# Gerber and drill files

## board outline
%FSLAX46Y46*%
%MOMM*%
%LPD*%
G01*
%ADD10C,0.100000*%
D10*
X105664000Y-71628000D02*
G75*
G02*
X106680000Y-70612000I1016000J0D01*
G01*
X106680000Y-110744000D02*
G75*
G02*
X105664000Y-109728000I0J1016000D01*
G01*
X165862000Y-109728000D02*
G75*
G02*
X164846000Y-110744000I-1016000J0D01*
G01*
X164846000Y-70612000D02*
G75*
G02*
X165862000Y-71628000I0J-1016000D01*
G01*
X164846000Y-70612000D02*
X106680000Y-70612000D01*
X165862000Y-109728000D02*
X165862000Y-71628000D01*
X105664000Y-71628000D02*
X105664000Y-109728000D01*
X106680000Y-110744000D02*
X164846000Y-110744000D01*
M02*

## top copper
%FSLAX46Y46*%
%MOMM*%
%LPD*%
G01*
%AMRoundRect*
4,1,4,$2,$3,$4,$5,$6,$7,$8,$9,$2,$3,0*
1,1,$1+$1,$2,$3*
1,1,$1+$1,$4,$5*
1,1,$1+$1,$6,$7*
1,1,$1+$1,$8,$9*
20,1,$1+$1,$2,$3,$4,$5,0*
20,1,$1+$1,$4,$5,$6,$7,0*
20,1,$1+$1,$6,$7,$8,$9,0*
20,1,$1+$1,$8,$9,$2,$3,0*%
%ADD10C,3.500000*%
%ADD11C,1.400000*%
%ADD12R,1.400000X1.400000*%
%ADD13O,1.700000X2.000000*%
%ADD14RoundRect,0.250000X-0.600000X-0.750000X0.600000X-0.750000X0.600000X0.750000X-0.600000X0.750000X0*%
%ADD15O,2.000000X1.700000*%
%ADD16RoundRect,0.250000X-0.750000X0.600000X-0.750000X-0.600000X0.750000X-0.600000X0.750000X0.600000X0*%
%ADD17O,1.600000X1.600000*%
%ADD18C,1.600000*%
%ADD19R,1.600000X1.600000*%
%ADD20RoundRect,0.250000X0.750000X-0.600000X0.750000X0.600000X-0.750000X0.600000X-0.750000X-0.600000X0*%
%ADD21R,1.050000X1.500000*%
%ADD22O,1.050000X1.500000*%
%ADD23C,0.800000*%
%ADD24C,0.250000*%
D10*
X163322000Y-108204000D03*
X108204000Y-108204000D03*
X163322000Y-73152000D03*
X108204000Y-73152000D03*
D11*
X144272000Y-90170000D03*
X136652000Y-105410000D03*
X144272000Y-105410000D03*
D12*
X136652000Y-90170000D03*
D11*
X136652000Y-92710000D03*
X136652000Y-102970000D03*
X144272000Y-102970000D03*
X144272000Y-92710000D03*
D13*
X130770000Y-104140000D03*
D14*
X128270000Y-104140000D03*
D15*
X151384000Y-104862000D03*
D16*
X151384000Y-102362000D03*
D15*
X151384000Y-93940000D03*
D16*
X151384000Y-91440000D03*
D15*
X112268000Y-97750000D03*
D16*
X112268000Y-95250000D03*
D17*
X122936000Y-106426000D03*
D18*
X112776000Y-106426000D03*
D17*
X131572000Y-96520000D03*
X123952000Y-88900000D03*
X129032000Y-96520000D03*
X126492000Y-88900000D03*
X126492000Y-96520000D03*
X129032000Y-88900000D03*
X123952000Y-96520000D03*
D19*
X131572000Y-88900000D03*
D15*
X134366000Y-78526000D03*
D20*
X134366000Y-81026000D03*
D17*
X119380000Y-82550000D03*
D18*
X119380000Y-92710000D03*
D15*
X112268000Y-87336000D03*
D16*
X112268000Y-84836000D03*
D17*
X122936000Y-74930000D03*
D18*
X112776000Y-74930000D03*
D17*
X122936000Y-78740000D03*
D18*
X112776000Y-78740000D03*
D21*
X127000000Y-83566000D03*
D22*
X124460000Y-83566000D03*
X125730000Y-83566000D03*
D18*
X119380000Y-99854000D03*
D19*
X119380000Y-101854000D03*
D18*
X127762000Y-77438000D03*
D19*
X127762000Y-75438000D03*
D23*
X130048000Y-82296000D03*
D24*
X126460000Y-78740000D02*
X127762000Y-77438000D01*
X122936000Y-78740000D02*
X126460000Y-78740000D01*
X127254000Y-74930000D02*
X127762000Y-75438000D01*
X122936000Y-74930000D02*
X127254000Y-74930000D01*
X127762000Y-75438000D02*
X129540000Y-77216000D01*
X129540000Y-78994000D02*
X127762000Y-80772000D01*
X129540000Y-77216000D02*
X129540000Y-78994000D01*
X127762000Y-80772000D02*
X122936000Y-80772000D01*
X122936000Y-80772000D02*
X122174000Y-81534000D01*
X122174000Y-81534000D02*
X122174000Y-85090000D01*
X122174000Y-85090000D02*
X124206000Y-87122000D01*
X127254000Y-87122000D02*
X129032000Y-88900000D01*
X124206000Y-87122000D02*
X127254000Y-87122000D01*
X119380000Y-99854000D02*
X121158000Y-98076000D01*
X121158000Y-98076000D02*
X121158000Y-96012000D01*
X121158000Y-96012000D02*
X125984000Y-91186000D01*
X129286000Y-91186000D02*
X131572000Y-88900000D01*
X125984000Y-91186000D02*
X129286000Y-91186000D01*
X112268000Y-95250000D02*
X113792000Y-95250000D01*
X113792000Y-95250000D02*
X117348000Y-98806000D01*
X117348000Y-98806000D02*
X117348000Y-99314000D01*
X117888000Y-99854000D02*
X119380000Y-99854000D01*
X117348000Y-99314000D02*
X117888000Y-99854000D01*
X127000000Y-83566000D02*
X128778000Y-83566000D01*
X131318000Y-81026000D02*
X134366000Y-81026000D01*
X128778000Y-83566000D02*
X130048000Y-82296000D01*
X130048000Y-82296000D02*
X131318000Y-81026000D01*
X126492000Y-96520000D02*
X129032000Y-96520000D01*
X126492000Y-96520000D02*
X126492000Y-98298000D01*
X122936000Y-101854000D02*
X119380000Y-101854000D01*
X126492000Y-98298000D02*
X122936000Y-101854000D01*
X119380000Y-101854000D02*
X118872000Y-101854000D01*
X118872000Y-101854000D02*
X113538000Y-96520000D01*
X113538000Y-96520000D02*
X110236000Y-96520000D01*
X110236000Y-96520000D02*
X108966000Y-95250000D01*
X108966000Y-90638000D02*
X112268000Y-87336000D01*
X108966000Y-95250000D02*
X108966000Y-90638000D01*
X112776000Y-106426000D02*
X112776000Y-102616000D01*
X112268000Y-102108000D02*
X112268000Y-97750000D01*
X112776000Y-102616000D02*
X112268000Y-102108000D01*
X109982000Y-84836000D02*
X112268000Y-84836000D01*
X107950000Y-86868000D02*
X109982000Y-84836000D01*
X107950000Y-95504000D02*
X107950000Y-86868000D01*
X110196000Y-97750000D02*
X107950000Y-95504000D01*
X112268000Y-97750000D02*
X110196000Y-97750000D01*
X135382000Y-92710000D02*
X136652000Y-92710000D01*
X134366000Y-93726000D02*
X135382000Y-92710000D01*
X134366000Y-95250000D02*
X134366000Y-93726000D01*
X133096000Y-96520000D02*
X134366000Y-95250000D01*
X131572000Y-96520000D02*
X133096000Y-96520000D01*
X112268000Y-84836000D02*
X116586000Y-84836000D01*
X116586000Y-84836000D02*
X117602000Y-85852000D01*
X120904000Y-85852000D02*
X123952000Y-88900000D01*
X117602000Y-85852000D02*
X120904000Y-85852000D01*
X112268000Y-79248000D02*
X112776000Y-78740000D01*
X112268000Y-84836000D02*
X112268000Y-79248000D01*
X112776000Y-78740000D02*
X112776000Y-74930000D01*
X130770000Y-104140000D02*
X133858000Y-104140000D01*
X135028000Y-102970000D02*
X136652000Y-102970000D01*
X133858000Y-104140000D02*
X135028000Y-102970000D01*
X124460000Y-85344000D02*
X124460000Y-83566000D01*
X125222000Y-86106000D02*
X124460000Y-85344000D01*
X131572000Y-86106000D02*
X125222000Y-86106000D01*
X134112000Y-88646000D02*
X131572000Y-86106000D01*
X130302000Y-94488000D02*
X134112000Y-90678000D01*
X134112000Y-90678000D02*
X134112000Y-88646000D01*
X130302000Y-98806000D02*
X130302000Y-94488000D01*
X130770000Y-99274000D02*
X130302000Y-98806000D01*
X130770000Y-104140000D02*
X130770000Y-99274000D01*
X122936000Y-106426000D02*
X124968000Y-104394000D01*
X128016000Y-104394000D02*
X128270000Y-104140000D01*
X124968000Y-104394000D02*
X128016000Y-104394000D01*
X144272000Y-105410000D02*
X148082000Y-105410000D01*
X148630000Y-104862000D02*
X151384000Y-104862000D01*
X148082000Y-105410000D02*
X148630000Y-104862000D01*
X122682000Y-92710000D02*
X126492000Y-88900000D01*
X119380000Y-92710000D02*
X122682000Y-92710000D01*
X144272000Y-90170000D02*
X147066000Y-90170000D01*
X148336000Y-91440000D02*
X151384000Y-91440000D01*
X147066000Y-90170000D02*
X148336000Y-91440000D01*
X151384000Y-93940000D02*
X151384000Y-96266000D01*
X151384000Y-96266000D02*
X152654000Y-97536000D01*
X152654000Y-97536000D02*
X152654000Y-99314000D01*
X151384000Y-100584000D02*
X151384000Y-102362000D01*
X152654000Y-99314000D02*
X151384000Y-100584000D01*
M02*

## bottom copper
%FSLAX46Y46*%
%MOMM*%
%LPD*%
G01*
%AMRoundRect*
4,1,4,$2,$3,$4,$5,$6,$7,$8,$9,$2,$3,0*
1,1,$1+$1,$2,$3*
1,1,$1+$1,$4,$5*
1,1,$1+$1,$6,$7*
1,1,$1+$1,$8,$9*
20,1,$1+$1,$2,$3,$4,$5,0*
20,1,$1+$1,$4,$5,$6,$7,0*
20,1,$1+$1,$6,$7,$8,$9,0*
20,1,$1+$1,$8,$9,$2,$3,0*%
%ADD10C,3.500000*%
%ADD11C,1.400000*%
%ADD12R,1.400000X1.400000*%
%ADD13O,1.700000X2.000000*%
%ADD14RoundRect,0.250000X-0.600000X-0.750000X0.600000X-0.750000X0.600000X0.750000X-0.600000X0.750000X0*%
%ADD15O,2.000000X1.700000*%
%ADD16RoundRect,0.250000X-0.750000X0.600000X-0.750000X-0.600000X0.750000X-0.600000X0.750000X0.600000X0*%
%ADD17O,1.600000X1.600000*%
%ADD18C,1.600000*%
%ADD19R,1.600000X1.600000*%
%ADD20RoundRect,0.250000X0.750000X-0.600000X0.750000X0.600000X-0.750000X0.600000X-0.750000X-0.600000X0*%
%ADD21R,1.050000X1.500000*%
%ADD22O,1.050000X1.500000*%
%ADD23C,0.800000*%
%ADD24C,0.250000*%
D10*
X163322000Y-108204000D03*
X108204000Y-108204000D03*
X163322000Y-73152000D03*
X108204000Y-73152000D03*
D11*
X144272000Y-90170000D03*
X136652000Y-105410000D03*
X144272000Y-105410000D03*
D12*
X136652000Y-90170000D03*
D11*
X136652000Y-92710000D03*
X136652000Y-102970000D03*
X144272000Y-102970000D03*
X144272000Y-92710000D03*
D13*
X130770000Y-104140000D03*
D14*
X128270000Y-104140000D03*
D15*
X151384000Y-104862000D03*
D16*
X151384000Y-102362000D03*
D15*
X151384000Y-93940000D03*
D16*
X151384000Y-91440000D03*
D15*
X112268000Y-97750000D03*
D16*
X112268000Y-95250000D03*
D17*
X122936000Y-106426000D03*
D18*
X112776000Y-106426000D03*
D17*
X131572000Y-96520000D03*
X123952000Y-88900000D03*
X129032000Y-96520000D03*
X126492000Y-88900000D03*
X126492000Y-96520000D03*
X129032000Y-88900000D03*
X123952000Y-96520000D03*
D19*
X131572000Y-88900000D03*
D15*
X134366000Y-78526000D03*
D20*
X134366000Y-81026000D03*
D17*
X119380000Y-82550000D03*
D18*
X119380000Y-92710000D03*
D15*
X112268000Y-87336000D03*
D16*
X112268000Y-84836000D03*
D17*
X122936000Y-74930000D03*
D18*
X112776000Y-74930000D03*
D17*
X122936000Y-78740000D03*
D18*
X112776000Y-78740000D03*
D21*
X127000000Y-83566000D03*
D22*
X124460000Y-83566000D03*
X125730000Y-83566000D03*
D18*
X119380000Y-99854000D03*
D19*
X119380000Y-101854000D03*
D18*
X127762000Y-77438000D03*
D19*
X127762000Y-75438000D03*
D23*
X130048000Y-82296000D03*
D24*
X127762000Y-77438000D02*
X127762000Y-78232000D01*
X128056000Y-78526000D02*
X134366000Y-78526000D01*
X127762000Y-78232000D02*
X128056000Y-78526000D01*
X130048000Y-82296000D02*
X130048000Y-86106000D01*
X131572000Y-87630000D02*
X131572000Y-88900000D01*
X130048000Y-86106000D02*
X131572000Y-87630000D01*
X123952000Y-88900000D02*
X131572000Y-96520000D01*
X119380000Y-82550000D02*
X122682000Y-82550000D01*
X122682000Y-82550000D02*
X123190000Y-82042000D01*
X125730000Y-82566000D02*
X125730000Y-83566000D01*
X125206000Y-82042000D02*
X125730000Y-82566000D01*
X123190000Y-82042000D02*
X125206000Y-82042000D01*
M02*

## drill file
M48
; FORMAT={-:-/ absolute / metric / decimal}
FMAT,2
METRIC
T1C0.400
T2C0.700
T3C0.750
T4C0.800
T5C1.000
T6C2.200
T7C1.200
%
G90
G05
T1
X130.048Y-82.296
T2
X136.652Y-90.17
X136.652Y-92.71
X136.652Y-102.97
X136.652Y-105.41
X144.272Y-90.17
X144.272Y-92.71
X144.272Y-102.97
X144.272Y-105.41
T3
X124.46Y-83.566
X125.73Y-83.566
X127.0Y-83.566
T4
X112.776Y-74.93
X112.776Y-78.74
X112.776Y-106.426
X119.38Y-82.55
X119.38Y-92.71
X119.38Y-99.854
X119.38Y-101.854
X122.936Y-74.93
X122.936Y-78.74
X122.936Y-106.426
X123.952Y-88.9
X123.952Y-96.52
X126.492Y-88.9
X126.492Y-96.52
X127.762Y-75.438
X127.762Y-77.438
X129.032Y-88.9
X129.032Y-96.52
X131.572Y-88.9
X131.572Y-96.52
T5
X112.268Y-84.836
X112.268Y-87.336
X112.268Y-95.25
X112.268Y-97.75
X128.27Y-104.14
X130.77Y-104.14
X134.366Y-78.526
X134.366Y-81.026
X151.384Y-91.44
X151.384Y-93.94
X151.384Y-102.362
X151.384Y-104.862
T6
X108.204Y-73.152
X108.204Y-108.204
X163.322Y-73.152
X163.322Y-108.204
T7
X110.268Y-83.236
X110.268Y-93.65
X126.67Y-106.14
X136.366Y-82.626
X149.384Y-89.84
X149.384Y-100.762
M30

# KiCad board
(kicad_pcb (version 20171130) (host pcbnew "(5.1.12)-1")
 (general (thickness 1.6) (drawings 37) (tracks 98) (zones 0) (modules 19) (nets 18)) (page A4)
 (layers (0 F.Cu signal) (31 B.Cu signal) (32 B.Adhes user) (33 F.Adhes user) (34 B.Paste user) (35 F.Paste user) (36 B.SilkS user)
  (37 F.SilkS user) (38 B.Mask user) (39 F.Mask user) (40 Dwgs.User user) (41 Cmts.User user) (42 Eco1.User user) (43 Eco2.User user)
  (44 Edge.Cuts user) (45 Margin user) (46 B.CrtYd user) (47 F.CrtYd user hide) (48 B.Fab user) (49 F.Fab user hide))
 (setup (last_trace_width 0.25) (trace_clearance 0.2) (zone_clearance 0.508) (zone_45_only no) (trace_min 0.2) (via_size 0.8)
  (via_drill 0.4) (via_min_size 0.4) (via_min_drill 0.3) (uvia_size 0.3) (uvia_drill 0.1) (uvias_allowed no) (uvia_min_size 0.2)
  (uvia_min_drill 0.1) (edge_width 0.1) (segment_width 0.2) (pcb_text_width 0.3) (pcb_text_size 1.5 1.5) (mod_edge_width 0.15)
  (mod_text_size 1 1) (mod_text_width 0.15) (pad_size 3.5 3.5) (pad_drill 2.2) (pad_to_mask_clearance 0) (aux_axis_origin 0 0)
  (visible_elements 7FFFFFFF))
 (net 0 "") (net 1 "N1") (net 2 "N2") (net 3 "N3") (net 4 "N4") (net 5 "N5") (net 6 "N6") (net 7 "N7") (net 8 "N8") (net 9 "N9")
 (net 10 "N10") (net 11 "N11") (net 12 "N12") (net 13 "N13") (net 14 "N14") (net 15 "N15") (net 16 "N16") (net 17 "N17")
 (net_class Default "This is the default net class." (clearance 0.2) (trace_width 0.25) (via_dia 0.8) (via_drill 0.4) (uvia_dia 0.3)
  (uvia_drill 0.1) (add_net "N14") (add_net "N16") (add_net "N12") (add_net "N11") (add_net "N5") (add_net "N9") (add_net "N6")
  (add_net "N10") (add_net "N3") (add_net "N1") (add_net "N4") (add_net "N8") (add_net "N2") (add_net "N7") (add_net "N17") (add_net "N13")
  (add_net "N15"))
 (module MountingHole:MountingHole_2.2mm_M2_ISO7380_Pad (layer F.Cu) (at 163.322 108.204)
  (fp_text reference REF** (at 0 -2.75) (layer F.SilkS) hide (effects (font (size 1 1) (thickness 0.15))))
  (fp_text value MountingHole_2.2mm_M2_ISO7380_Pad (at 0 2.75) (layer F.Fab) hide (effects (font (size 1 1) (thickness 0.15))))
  (pad 1 thru_hole circle (at 0 0) (size 3.5 3.5) (drill 2.2) (layers *.Cu *.Mask)))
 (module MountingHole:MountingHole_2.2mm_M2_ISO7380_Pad (layer F.Cu) (at 108.204 108.204)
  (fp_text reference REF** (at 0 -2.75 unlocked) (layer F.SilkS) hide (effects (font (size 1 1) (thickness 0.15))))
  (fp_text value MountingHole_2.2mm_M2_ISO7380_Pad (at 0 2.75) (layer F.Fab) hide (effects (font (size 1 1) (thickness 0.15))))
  (pad 1 thru_hole circle (at 0 0) (size 3.5 3.5) (drill 2.2) (layers *.Cu *.Mask)))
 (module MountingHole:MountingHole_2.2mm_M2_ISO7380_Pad (layer F.Cu) (at 163.322 73.152)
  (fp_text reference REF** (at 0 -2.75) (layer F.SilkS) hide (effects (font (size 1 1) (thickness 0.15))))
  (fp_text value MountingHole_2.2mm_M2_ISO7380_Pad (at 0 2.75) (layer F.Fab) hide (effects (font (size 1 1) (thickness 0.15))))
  (pad 1 thru_hole circle (at 0 0) (size 3.5 3.5) (drill 2.2) (layers *.Cu *.Mask)))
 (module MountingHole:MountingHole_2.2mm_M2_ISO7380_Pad (layer F.Cu) (at 108.204 73.152)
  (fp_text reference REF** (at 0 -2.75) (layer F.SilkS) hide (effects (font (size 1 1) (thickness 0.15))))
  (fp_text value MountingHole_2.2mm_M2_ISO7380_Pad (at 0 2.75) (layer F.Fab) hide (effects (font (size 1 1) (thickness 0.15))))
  (pad 1 thru_hole circle (at 0 0) (size 3.5 3.5) (drill 2.2) (layers *.Cu *.Mask)))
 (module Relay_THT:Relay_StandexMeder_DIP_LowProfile (layer F.Cu) (at 136.652 90.17)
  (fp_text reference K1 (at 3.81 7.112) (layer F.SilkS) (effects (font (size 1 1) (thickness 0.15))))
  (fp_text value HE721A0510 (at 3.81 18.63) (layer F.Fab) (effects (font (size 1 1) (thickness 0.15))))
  (pad 14 thru_hole circle (at 7.62 0) (size 1.4 1.4) (drill 0.7) (layers *.Cu *.Mask) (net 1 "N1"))
  (pad 7 thru_hole circle (at 0 15.24) (size 1.4 1.4) (drill 0.7) (layers *.Cu *.Mask) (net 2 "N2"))
  (pad 8 thru_hole circle (at 7.62 15.24) (size 1.4 1.4) (drill 0.7) (layers *.Cu *.Mask) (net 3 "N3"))
  (pad 1 thru_hole rect (at 0 0) (size 1.4 1.4) (drill 0.7) (layers *.Cu *.Mask) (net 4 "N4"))
  (pad 2 thru_hole circle (at 0 2.54) (size 1.4 1.4) (drill 0.7) (layers *.Cu *.Mask) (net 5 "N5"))
  (pad 6 thru_hole circle (at 0 12.8) (size 1.4 1.4) (drill 0.7) (layers *.Cu *.Mask) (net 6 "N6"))
  (pad 9 thru_hole circle (at 7.62 12.8) (size 1.4 1.4) (drill 0.7) (layers *.Cu *.Mask) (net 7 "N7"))
  (pad 13 thru_hole circle (at 7.62 2.54) (size 1.4 1.4) (drill 0.7) (layers *.Cu *.Mask) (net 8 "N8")))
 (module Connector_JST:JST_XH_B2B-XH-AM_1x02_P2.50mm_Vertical (layer F.Cu) (at 128.27 104.14)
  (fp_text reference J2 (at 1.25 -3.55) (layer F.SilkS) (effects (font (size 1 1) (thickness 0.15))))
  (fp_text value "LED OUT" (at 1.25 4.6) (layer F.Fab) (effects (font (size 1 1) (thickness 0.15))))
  (pad "" np_thru_hole circle (at -1.6 2) (size 1.2 1.2) (drill 1.2) (layers *.Cu *.Mask))
  (pad 2 thru_hole oval (at 2.5 0) (size 1.7 2) (drill 1) (layers *.Cu *.Mask) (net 6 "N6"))
  (pad 1 thru_hole roundrect (at 0 0) (size 1.7 2) (drill 1) (layers *.Cu *.Mask) (roundrect_rratio 0.147059) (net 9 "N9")))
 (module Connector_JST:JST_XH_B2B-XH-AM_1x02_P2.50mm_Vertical (layer F.Cu) (at 151.384 102.362 270)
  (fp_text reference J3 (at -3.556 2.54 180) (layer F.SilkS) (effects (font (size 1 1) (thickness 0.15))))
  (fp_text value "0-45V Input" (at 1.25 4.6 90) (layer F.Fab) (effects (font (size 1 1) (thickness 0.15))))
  (pad "" np_thru_hole circle (at -1.6 2 270) (size 1.2 1.2) (drill 1.2) (layers *.Cu *.Mask))
  (pad 2 thru_hole oval (at 2.5 0 270) (size 1.7 2) (drill 1) (layers *.Cu *.Mask) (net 3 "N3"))
  (pad 1 thru_hole roundrect (at 0 0 270) (size 1.7 2) (drill 1) (layers *.Cu *.Mask) (roundrect_rratio 0.147059) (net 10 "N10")))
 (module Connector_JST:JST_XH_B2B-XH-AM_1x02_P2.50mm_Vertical (layer F.Cu) (at 151.384 91.44 270)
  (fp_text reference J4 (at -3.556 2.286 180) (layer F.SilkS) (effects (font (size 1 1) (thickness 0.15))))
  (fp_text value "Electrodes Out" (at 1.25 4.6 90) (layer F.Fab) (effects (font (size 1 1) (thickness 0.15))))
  (pad "" np_thru_hole circle (at -1.6 2 270) (size 1.2 1.2) (drill 1.2) (layers *.Cu *.Mask))
  (pad 2 thru_hole oval (at 2.5 0 270) (size 1.7 2) (drill 1) (layers *.Cu *.Mask) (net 10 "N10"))
  (pad 1 thru_hole roundrect (at 0 0 270) (size 1.7 2) (drill 1) (layers *.Cu *.Mask) (roundrect_rratio 0.147059) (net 1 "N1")))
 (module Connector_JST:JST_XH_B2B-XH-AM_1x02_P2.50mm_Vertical (layer F.Cu) (at 112.268 95.25 270)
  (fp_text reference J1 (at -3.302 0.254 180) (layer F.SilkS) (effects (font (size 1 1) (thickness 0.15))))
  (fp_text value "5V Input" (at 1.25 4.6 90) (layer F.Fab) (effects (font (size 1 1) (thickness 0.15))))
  (pad "" np_thru_hole circle (at -1.6 2 270) (size 1.2 1.2) (drill 1.2) (layers *.Cu *.Mask))
  (pad 2 thru_hole oval (at 2.5 0 270) (size 1.7 2) (drill 1) (layers *.Cu *.Mask) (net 5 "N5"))
  (pad 1 thru_hole roundrect (at 0 0 270) (size 1.7 2) (drill 1) (layers *.Cu *.Mask) (roundrect_rratio 0.147059) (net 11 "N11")))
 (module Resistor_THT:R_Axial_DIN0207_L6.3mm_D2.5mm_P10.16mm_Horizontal (layer F.Cu) (at 112.776 106.426)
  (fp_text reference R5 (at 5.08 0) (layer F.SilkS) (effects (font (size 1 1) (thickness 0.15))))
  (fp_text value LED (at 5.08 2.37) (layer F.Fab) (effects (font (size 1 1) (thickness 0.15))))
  (pad 2 thru_hole oval (at 10.16 0) (size 1.6 1.6) (drill 0.8) (layers *.Cu *.Mask) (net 9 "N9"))
  (pad 1 thru_hole circle (at 0 0) (size 1.6 1.6) (drill 0.8) (layers *.Cu *.Mask) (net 5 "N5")))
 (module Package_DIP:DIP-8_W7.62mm (layer F.Cu) (at 131.572 88.9 270)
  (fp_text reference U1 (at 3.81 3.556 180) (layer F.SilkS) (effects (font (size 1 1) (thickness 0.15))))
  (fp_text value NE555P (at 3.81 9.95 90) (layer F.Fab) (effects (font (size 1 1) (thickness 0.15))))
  (pad 8 thru_hole oval (at 7.62 0 270) (size 1.6 1.6) (drill 0.8) (layers *.Cu *.Mask) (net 5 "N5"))
  (pad 4 thru_hole oval (at 0 7.62 270) (size 1.6 1.6) (drill 0.8) (layers *.Cu *.Mask) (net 5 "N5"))
  (pad 7 thru_hole oval (at 7.62 2.54 270) (size 1.6 1.6) (drill 0.8) (layers *.Cu *.Mask) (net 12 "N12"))
  (pad 3 thru_hole oval (at 0 5.08 270) (size 1.6 1.6) (drill 0.8) (layers *.Cu *.Mask) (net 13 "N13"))
  (pad 6 thru_hole oval (at 7.62 5.08 270) (size 1.6 1.6) (drill 0.8) (layers *.Cu *.Mask) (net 12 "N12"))
  (pad 2 thru_hole oval (at 0 2.54 270) (size 1.6 1.6) (drill 0.8) (layers *.Cu *.Mask) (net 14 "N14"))
  (pad 5 thru_hole oval (at 7.62 7.62 270) (size 1.6 1.6) (drill 0.8) (layers *.Cu *.Mask) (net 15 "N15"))
  (pad 1 thru_hole rect (at 0 0 270) (size 1.6 1.6) (drill 0.8) (layers *.Cu *.Mask) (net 11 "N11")))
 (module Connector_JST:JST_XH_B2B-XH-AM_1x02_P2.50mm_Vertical (layer F.Cu) (at 134.366 81.026 90)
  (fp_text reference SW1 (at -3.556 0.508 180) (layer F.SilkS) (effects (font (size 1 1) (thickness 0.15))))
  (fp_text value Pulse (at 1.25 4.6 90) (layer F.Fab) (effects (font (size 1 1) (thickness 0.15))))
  (pad "" np_thru_hole circle (at -1.6 2 90) (size 1.2 1.2) (drill 1.2) (layers *.Cu *.Mask))
  (pad 2 thru_hole oval (at 2.5 0 90) (size 1.7 2) (drill 1) (layers *.Cu *.Mask) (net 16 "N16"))
  (pad 1 thru_hole roundrect (at 0 0 90) (size 1.7 2) (drill 1) (layers *.Cu *.Mask) (roundrect_rratio 0.147059) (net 11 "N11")))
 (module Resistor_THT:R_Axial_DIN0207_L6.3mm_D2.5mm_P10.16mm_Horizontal (layer F.Cu) (at 119.38 92.71 90)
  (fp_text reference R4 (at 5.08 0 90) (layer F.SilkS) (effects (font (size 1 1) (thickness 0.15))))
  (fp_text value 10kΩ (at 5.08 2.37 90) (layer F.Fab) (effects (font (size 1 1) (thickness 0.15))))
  (pad 2 thru_hole oval (at 10.16 0 90) (size 1.6 1.6) (drill 0.8) (layers *.Cu *.Mask) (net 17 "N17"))
  (pad 1 thru_hole circle (at 0 0 90) (size 1.6 1.6) (drill 0.8) (layers *.Cu *.Mask) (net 13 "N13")))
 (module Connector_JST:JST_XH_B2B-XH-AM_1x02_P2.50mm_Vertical (layer F.Cu) (at 112.268 84.836 270)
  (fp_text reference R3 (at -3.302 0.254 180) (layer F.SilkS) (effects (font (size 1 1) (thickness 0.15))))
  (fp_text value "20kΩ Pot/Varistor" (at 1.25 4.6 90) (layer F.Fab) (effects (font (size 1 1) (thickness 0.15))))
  (pad "" np_thru_hole circle (at -1.6 2 270) (size 1.2 1.2) (drill 1.2) (layers *.Cu *.Mask))
  (pad 2 thru_hole oval (at 2.5 0 270) (size 1.7 2) (drill 1) (layers *.Cu *.Mask) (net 12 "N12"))
  (pad 1 thru_hole roundrect (at 0 0 270) (size 1.7 2) (drill 1) (layers *.Cu *.Mask) (roundrect_rratio 0.147059) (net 5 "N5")))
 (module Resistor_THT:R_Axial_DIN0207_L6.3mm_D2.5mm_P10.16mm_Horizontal (layer F.Cu) (at 112.776 74.93)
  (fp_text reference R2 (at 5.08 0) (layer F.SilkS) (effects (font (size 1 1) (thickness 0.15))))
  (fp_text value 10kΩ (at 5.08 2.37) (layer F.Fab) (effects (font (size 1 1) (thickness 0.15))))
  (pad 2 thru_hole oval (at 10.16 0) (size 1.6 1.6) (drill 0.8) (layers *.Cu *.Mask) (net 14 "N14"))
  (pad 1 thru_hole circle (at 0 0) (size 1.6 1.6) (drill 0.8) (layers *.Cu *.Mask) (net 5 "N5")))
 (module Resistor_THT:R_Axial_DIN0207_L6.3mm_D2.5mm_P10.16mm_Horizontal (layer F.Cu) (at 112.776 78.74)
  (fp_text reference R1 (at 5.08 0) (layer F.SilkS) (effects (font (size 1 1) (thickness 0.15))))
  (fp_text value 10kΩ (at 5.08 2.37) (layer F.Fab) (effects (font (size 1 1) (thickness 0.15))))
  (pad 2 thru_hole oval (at 10.16 0) (size 1.6 1.6) (drill 0.8) (layers *.Cu *.Mask) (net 16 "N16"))
  (pad 1 thru_hole circle (at 0 0) (size 1.6 1.6) (drill 0.8) (layers *.Cu *.Mask) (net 5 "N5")))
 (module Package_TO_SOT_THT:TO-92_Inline (layer F.Cu) (at 127 83.566 180)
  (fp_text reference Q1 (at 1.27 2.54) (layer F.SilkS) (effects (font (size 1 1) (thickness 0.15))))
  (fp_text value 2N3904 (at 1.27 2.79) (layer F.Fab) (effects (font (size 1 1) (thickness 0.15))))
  (pad 1 thru_hole rect (at 0 0 180) (size 1.05 1.5) (drill 0.75) (layers *.Cu *.Mask) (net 11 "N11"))
  (pad 3 thru_hole oval (at 2.54 0 180) (size 1.05 1.5) (drill 0.75) (layers *.Cu *.Mask) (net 6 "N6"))
  (pad 2 thru_hole oval (at 1.27 0 180) (size 1.05 1.5) (drill 0.75) (layers *.Cu *.Mask) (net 17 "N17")))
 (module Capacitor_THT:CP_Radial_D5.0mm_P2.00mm (layer F.Cu) (at 119.38 101.854 90)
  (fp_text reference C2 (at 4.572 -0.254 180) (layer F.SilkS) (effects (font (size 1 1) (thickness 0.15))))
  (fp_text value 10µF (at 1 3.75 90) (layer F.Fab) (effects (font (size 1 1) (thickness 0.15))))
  (pad 2 thru_hole circle (at 2 0 90) (size 1.6 1.6) (drill 0.8) (layers *.Cu *.Mask) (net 11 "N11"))
  (pad 1 thru_hole rect (at 0 0 90) (size 1.6 1.6) (drill 0.8) (layers *.Cu *.Mask) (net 12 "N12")))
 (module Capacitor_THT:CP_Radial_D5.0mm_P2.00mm (layer F.Cu) (at 127.762 75.438 270)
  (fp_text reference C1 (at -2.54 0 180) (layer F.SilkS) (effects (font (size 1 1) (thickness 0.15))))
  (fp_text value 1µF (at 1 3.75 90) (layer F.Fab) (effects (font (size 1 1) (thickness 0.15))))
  (pad 2 thru_hole circle (at 2 0 270) (size 1.6 1.6) (drill 0.8) (layers *.Cu *.Mask) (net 16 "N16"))
  (pad 1 thru_hole rect (at 0 0 270) (size 1.6 1.6) (drill 0.8) (layers *.Cu *.Mask) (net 14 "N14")))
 (gr_arc (start 106.68 71.628) (end 106.68 70.612) (angle -90) (layer Edge.Cuts) (width 0.1))
 (gr_arc (start 106.68 109.728) (end 105.664 109.728) (angle -90) (layer Edge.Cuts) (width 0.1))
 (gr_arc (start 164.846 109.728) (end 164.846 110.744) (angle -90) (layer Edge.Cuts) (width 0.1))
 (gr_arc (start 164.846 71.628) (end 165.862 71.628) (angle -90) (layer Edge.Cuts) (width 0.1))
 (gr_line (start 164.846 70.612) (end 106.68 70.612) (layer Edge.Cuts) (width 0.1))
 (gr_line (start 165.862 109.728) (end 165.862 71.628) (layer Edge.Cuts) (width 0.1))
 (gr_line (start 105.664 71.628) (end 105.664 109.728) (layer Edge.Cuts) (width 0.1))
 (gr_line (start 106.68 110.744) (end 164.846 110.744) (layer Edge.Cuts) (width 0.1))
 (segment (start 126.46 78.74) (end 127.762 77.438) (width 0.25) (layer F.Cu) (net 16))
 (segment (start 122.936 78.74) (end 126.46 78.74) (width 0.25) (layer F.Cu) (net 16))
 (segment (start 127.762 77.438) (end 127.762 78.232) (width 0.25) (layer B.Cu) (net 16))
 (segment (start 128.056 78.526) (end 134.366 78.526) (width 0.25) (layer B.Cu) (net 16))
 (segment (start 127.762 78.232) (end 128.056 78.526) (width 0.25) (layer B.Cu) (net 16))
 (segment (start 127.254 74.93) (end 127.762 75.438) (width 0.25) (layer F.Cu) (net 14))
 (segment (start 122.936 74.93) (end 127.254 74.93) (width 0.25) (layer F.Cu) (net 14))
 (segment (start 127.762 75.438) (end 129.54 77.216) (width 0.25) (layer F.Cu) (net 14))
 (segment (start 129.54 78.994) (end 127.762 80.772) (width 0.25) (layer F.Cu) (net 14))
 (segment (start 129.54 77.216) (end 129.54 78.994) (width 0.25) (layer F.Cu) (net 14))
 (segment (start 127.762 80.772) (end 122.936 80.772) (width 0.25) (layer F.Cu) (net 14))
 (segment (start 122.936 80.772) (end 122.174 81.534) (width 0.25) (layer F.Cu) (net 14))
 (segment (start 122.174 81.534) (end 122.174 85.09) (width 0.25) (layer F.Cu) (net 14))
 (segment (start 122.174 85.09) (end 124.206 87.122) (width 0.25) (layer F.Cu) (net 14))
 (segment (start 127.254 87.122) (end 129.032 88.9) (width 0.25) (layer F.Cu) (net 14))
 (segment (start 124.206 87.122) (end 127.254 87.122) (width 0.25) (layer F.Cu) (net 14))
 (segment (start 119.38 99.854) (end 121.158 98.076) (width 0.25) (layer F.Cu) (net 11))
 (segment (start 121.158 98.076) (end 121.158 96.012) (width 0.25) (layer F.Cu) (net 11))
 (segment (start 121.158 96.012) (end 125.984 91.186) (width 0.25) (layer F.Cu) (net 11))
 (segment (start 129.286 91.186) (end 131.572 88.9) (width 0.25) (layer F.Cu) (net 11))
 (segment (start 125.984 91.186) (end 129.286 91.186) (width 0.25) (layer F.Cu) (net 11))
 (segment (start 112.268 95.25) (end 113.792 95.25) (width 0.25) (layer F.Cu) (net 11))
 (segment (start 113.792 95.25) (end 117.348 98.806) (width 0.25) (layer F.Cu) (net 11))
 (segment (start 117.348 98.806) (end 117.348 99.314) (width 0.25) (layer F.Cu) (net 11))
 (segment (start 117.888 99.854) (end 119.38 99.854) (width 0.25) (layer F.Cu) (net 11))
 (segment (start 117.348 99.314) (end 117.888 99.854) (width 0.25) (layer F.Cu) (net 11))
 (segment (start 127 83.566) (end 128.778 83.566) (width 0.25) (layer F.Cu) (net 11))
 (segment (start 131.318 81.026) (end 134.366 81.026) (width 0.25) (layer F.Cu) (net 11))
 (segment (start 128.778 83.566) (end 130.048 82.296) (width 0.25) (layer F.Cu) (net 11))
 (segment (start 130.048 82.296) (end 131.318 81.026) (width 0.25) (layer F.Cu) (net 11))
 (via (at 130.048 82.296) (size 0.8) (drill 0.4) (layers F.Cu B.Cu) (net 11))
 (segment (start 130.048 82.296) (end 130.048 86.106) (width 0.25) (layer B.Cu) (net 11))
 (segment (start 131.572 87.63) (end 131.572 88.9) (width 0.25) (layer B.Cu) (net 11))
 (segment (start 130.048 86.106) (end 131.572 87.63) (width 0.25) (layer B.Cu) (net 11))
 (segment (start 126.492 96.52) (end 129.032 96.52) (width 0.25) (layer F.Cu) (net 12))
 (segment (start 126.492 96.52) (end 126.492 98.298) (width 0.25) (layer F.Cu) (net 12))
 (segment (start 122.936 101.854) (end 119.38 101.854) (width 0.25) (layer F.Cu) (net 12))
 (segment (start 126.492 98.298) (end 122.936 101.854) (width 0.25) (layer F.Cu) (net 12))
 (segment (start 119.38 101.854) (end 118.872 101.854) (width 0.25) (layer F.Cu) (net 12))
 (segment (start 118.872 101.854) (end 113.538 96.52) (width 0.25) (layer F.Cu) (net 12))
 (segment (start 113.538 96.52) (end 110.236 96.52) (width 0.25) (layer F.Cu) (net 12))
 (segment (start 110.236 96.52) (end 108.966 95.25) (width 0.25) (layer F.Cu) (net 12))
 (segment (start 108.966 90.638) (end 112.268 87.336) (width 0.25) (layer F.Cu) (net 12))
 (segment (start 108.966 95.25) (end 108.966 90.638) (width 0.25) (layer F.Cu) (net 12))
 (segment (start 112.776 106.426) (end 112.776 102.616) (width 0.25) (layer F.Cu) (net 5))
 (segment (start 112.268 102.108) (end 112.268 97.75) (width 0.25) (layer F.Cu) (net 5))
 (segment (start 112.776 102.616) (end 112.268 102.108) (width 0.25) (layer F.Cu) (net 5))
 (segment (start 109.982 84.836) (end 112.268 84.836) (width 0.25) (layer F.Cu) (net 5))
 (segment (start 107.95 86.868) (end 109.982 84.836) (width 0.25) (layer F.Cu) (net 5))
 (segment (start 107.95 95.504) (end 107.95 86.868) (width 0.25) (layer F.Cu) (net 5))
 (segment (start 110.196 97.75) (end 107.95 95.504) (width 0.25) (layer F.Cu) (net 5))
 (segment (start 112.268 97.75) (end 110.196 97.75) (width 0.25) (layer F.Cu) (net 5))
 (segment (start 135.382 92.71) (end 136.652 92.71) (width 0.25) (layer F.Cu) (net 5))
 (segment (start 134.366 93.726) (end 135.382 92.71) (width 0.25) (layer F.Cu) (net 5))
 (segment (start 134.366 95.25) (end 134.366 93.726) (width 0.25) (layer F.Cu) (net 5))
 (segment (start 133.096 96.52) (end 134.366 95.25) (width 0.25) (layer F.Cu) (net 5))
 (segment (start 131.572 96.52) (end 133.096 96.52) (width 0.25) (layer F.Cu) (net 5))
 (segment (start 112.268 84.836) (end 116.586 84.836) (width 0.25) (layer F.Cu) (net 5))
 (segment (start 116.586 84.836) (end 117.602 85.852) (width 0.25) (layer F.Cu) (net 5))
 (segment (start 120.904 85.852) (end 123.952 88.9) (width 0.25) (layer F.Cu) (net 5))
 (segment (start 117.602 85.852) (end 120.904 85.852) (width 0.25) (layer F.Cu) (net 5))
 (segment (start 112.268 79.248) (end 112.776 78.74) (width 0.25) (layer F.Cu) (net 5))
 (segment (start 112.268 84.836) (end 112.268 79.248) (width 0.25) (layer F.Cu) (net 5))
 (segment (start 112.776 78.74) (end 112.776 74.93) (width 0.25) (layer F.Cu) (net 5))
 (segment (start 123.952 88.9) (end 131.572 96.52) (width 0.25) (layer B.Cu) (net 5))
 (segment (start 130.77 104.14) (end 133.858 104.14) (width 0.25) (layer F.Cu) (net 6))
 (segment (start 135.028 102.97) (end 136.652 102.97) (width 0.25) (layer F.Cu) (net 6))
 (segment (start 133.858 104.14) (end 135.028 102.97) (width 0.25) (layer F.Cu) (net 6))
 (segment (start 124.46 85.344) (end 124.46 83.566) (width 0.25) (layer F.Cu) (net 6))
 (segment (start 125.222 86.106) (end 124.46 85.344) (width 0.25) (layer F.Cu) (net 6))
 (segment (start 131.572 86.106) (end 125.222 86.106) (width 0.25) (layer F.Cu) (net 6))
 (segment (start 134.112 88.646) (end 131.572 86.106) (width 0.25) (layer F.Cu) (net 6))
 (segment (start 130.302 94.488) (end 134.112 90.678) (width 0.25) (layer F.Cu) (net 6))
 (segment (start 134.112 90.678) (end 134.112 88.646) (width 0.25) (layer F.Cu) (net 6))
 (segment (start 130.302 98.806) (end 130.302 94.488) (width 0.25) (layer F.Cu) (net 6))
 (segment (start 130.77 99.274) (end 130.302 98.806) (width 0.25) (layer F.Cu) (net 6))
 (segment (start 130.77 104.14) (end 130.77 99.274) (width 0.25) (layer F.Cu) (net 6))
 (segment (start 122.936 106.426) (end 124.968 104.394) (width 0.25) (layer F.Cu) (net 9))
 (segment (start 128.016 104.394) (end 128.27 104.14) (width 0.25) (layer F.Cu) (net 9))
 (segment (start 124.968 104.394) (end 128.016 104.394) (width 0.25) (layer F.Cu) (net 9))
 (segment (start 144.272 105.41) (end 148.082 105.41) (width 0.25) (layer F.Cu) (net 3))
 (segment (start 148.63 104.862) (end 151.384 104.862) (width 0.25) (layer F.Cu) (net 3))
 (segment (start 148.082 105.41) (end 148.63 104.862) (width 0.25) (layer F.Cu) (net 3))
 (segment (start 119.38 82.55) (end 122.682 82.55) (width 0.25) (layer B.Cu) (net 17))
 (segment (start 122.682 82.55) (end 123.19 82.042) (width 0.25) (layer B.Cu) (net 17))
 (segment (start 125.73 82.566) (end 125.73 83.566) (width 0.25) (layer B.Cu) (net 17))
 (segment (start 125.206 82.042) (end 125.73 82.566) (width 0.25) (layer B.Cu) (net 17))
 (segment (start 123.19 82.042) (end 125.206 82.042) (width 0.25) (layer B.Cu) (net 17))
 (segment (start 122.682 92.71) (end 126.492 88.9) (width 0.25) (layer F.Cu) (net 13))
 (segment (start 119.38 92.71) (end 122.682 92.71) (width 0.25) (layer F.Cu) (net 13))
 (segment (start 144.272 90.17) (end 147.066 90.17) (width 0.25) (layer F.Cu) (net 1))
 (segment (start 148.336 91.44) (end 151.384 91.44) (width 0.25) (layer F.Cu) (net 1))
 (segment (start 147.066 90.17) (end 148.336 91.44) (width 0.25) (layer F.Cu) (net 1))
 (segment (start 151.384 93.94) (end 151.384 96.266) (width 0.25) (layer F.Cu) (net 10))
 (segment (start 151.384 96.266) (end 152.654 97.536) (width 0.25) (layer F.Cu) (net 10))
 (segment (start 152.654 97.536) (end 152.654 99.314) (width 0.25) (layer F.Cu) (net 10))
 (segment (start 151.384 100.584) (end 151.384 102.362) (width 0.25) (layer F.Cu) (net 10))
 (segment (start 152.654 99.314) (end 151.384 100.584) (width 0.25) (layer F.Cu) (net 10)))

